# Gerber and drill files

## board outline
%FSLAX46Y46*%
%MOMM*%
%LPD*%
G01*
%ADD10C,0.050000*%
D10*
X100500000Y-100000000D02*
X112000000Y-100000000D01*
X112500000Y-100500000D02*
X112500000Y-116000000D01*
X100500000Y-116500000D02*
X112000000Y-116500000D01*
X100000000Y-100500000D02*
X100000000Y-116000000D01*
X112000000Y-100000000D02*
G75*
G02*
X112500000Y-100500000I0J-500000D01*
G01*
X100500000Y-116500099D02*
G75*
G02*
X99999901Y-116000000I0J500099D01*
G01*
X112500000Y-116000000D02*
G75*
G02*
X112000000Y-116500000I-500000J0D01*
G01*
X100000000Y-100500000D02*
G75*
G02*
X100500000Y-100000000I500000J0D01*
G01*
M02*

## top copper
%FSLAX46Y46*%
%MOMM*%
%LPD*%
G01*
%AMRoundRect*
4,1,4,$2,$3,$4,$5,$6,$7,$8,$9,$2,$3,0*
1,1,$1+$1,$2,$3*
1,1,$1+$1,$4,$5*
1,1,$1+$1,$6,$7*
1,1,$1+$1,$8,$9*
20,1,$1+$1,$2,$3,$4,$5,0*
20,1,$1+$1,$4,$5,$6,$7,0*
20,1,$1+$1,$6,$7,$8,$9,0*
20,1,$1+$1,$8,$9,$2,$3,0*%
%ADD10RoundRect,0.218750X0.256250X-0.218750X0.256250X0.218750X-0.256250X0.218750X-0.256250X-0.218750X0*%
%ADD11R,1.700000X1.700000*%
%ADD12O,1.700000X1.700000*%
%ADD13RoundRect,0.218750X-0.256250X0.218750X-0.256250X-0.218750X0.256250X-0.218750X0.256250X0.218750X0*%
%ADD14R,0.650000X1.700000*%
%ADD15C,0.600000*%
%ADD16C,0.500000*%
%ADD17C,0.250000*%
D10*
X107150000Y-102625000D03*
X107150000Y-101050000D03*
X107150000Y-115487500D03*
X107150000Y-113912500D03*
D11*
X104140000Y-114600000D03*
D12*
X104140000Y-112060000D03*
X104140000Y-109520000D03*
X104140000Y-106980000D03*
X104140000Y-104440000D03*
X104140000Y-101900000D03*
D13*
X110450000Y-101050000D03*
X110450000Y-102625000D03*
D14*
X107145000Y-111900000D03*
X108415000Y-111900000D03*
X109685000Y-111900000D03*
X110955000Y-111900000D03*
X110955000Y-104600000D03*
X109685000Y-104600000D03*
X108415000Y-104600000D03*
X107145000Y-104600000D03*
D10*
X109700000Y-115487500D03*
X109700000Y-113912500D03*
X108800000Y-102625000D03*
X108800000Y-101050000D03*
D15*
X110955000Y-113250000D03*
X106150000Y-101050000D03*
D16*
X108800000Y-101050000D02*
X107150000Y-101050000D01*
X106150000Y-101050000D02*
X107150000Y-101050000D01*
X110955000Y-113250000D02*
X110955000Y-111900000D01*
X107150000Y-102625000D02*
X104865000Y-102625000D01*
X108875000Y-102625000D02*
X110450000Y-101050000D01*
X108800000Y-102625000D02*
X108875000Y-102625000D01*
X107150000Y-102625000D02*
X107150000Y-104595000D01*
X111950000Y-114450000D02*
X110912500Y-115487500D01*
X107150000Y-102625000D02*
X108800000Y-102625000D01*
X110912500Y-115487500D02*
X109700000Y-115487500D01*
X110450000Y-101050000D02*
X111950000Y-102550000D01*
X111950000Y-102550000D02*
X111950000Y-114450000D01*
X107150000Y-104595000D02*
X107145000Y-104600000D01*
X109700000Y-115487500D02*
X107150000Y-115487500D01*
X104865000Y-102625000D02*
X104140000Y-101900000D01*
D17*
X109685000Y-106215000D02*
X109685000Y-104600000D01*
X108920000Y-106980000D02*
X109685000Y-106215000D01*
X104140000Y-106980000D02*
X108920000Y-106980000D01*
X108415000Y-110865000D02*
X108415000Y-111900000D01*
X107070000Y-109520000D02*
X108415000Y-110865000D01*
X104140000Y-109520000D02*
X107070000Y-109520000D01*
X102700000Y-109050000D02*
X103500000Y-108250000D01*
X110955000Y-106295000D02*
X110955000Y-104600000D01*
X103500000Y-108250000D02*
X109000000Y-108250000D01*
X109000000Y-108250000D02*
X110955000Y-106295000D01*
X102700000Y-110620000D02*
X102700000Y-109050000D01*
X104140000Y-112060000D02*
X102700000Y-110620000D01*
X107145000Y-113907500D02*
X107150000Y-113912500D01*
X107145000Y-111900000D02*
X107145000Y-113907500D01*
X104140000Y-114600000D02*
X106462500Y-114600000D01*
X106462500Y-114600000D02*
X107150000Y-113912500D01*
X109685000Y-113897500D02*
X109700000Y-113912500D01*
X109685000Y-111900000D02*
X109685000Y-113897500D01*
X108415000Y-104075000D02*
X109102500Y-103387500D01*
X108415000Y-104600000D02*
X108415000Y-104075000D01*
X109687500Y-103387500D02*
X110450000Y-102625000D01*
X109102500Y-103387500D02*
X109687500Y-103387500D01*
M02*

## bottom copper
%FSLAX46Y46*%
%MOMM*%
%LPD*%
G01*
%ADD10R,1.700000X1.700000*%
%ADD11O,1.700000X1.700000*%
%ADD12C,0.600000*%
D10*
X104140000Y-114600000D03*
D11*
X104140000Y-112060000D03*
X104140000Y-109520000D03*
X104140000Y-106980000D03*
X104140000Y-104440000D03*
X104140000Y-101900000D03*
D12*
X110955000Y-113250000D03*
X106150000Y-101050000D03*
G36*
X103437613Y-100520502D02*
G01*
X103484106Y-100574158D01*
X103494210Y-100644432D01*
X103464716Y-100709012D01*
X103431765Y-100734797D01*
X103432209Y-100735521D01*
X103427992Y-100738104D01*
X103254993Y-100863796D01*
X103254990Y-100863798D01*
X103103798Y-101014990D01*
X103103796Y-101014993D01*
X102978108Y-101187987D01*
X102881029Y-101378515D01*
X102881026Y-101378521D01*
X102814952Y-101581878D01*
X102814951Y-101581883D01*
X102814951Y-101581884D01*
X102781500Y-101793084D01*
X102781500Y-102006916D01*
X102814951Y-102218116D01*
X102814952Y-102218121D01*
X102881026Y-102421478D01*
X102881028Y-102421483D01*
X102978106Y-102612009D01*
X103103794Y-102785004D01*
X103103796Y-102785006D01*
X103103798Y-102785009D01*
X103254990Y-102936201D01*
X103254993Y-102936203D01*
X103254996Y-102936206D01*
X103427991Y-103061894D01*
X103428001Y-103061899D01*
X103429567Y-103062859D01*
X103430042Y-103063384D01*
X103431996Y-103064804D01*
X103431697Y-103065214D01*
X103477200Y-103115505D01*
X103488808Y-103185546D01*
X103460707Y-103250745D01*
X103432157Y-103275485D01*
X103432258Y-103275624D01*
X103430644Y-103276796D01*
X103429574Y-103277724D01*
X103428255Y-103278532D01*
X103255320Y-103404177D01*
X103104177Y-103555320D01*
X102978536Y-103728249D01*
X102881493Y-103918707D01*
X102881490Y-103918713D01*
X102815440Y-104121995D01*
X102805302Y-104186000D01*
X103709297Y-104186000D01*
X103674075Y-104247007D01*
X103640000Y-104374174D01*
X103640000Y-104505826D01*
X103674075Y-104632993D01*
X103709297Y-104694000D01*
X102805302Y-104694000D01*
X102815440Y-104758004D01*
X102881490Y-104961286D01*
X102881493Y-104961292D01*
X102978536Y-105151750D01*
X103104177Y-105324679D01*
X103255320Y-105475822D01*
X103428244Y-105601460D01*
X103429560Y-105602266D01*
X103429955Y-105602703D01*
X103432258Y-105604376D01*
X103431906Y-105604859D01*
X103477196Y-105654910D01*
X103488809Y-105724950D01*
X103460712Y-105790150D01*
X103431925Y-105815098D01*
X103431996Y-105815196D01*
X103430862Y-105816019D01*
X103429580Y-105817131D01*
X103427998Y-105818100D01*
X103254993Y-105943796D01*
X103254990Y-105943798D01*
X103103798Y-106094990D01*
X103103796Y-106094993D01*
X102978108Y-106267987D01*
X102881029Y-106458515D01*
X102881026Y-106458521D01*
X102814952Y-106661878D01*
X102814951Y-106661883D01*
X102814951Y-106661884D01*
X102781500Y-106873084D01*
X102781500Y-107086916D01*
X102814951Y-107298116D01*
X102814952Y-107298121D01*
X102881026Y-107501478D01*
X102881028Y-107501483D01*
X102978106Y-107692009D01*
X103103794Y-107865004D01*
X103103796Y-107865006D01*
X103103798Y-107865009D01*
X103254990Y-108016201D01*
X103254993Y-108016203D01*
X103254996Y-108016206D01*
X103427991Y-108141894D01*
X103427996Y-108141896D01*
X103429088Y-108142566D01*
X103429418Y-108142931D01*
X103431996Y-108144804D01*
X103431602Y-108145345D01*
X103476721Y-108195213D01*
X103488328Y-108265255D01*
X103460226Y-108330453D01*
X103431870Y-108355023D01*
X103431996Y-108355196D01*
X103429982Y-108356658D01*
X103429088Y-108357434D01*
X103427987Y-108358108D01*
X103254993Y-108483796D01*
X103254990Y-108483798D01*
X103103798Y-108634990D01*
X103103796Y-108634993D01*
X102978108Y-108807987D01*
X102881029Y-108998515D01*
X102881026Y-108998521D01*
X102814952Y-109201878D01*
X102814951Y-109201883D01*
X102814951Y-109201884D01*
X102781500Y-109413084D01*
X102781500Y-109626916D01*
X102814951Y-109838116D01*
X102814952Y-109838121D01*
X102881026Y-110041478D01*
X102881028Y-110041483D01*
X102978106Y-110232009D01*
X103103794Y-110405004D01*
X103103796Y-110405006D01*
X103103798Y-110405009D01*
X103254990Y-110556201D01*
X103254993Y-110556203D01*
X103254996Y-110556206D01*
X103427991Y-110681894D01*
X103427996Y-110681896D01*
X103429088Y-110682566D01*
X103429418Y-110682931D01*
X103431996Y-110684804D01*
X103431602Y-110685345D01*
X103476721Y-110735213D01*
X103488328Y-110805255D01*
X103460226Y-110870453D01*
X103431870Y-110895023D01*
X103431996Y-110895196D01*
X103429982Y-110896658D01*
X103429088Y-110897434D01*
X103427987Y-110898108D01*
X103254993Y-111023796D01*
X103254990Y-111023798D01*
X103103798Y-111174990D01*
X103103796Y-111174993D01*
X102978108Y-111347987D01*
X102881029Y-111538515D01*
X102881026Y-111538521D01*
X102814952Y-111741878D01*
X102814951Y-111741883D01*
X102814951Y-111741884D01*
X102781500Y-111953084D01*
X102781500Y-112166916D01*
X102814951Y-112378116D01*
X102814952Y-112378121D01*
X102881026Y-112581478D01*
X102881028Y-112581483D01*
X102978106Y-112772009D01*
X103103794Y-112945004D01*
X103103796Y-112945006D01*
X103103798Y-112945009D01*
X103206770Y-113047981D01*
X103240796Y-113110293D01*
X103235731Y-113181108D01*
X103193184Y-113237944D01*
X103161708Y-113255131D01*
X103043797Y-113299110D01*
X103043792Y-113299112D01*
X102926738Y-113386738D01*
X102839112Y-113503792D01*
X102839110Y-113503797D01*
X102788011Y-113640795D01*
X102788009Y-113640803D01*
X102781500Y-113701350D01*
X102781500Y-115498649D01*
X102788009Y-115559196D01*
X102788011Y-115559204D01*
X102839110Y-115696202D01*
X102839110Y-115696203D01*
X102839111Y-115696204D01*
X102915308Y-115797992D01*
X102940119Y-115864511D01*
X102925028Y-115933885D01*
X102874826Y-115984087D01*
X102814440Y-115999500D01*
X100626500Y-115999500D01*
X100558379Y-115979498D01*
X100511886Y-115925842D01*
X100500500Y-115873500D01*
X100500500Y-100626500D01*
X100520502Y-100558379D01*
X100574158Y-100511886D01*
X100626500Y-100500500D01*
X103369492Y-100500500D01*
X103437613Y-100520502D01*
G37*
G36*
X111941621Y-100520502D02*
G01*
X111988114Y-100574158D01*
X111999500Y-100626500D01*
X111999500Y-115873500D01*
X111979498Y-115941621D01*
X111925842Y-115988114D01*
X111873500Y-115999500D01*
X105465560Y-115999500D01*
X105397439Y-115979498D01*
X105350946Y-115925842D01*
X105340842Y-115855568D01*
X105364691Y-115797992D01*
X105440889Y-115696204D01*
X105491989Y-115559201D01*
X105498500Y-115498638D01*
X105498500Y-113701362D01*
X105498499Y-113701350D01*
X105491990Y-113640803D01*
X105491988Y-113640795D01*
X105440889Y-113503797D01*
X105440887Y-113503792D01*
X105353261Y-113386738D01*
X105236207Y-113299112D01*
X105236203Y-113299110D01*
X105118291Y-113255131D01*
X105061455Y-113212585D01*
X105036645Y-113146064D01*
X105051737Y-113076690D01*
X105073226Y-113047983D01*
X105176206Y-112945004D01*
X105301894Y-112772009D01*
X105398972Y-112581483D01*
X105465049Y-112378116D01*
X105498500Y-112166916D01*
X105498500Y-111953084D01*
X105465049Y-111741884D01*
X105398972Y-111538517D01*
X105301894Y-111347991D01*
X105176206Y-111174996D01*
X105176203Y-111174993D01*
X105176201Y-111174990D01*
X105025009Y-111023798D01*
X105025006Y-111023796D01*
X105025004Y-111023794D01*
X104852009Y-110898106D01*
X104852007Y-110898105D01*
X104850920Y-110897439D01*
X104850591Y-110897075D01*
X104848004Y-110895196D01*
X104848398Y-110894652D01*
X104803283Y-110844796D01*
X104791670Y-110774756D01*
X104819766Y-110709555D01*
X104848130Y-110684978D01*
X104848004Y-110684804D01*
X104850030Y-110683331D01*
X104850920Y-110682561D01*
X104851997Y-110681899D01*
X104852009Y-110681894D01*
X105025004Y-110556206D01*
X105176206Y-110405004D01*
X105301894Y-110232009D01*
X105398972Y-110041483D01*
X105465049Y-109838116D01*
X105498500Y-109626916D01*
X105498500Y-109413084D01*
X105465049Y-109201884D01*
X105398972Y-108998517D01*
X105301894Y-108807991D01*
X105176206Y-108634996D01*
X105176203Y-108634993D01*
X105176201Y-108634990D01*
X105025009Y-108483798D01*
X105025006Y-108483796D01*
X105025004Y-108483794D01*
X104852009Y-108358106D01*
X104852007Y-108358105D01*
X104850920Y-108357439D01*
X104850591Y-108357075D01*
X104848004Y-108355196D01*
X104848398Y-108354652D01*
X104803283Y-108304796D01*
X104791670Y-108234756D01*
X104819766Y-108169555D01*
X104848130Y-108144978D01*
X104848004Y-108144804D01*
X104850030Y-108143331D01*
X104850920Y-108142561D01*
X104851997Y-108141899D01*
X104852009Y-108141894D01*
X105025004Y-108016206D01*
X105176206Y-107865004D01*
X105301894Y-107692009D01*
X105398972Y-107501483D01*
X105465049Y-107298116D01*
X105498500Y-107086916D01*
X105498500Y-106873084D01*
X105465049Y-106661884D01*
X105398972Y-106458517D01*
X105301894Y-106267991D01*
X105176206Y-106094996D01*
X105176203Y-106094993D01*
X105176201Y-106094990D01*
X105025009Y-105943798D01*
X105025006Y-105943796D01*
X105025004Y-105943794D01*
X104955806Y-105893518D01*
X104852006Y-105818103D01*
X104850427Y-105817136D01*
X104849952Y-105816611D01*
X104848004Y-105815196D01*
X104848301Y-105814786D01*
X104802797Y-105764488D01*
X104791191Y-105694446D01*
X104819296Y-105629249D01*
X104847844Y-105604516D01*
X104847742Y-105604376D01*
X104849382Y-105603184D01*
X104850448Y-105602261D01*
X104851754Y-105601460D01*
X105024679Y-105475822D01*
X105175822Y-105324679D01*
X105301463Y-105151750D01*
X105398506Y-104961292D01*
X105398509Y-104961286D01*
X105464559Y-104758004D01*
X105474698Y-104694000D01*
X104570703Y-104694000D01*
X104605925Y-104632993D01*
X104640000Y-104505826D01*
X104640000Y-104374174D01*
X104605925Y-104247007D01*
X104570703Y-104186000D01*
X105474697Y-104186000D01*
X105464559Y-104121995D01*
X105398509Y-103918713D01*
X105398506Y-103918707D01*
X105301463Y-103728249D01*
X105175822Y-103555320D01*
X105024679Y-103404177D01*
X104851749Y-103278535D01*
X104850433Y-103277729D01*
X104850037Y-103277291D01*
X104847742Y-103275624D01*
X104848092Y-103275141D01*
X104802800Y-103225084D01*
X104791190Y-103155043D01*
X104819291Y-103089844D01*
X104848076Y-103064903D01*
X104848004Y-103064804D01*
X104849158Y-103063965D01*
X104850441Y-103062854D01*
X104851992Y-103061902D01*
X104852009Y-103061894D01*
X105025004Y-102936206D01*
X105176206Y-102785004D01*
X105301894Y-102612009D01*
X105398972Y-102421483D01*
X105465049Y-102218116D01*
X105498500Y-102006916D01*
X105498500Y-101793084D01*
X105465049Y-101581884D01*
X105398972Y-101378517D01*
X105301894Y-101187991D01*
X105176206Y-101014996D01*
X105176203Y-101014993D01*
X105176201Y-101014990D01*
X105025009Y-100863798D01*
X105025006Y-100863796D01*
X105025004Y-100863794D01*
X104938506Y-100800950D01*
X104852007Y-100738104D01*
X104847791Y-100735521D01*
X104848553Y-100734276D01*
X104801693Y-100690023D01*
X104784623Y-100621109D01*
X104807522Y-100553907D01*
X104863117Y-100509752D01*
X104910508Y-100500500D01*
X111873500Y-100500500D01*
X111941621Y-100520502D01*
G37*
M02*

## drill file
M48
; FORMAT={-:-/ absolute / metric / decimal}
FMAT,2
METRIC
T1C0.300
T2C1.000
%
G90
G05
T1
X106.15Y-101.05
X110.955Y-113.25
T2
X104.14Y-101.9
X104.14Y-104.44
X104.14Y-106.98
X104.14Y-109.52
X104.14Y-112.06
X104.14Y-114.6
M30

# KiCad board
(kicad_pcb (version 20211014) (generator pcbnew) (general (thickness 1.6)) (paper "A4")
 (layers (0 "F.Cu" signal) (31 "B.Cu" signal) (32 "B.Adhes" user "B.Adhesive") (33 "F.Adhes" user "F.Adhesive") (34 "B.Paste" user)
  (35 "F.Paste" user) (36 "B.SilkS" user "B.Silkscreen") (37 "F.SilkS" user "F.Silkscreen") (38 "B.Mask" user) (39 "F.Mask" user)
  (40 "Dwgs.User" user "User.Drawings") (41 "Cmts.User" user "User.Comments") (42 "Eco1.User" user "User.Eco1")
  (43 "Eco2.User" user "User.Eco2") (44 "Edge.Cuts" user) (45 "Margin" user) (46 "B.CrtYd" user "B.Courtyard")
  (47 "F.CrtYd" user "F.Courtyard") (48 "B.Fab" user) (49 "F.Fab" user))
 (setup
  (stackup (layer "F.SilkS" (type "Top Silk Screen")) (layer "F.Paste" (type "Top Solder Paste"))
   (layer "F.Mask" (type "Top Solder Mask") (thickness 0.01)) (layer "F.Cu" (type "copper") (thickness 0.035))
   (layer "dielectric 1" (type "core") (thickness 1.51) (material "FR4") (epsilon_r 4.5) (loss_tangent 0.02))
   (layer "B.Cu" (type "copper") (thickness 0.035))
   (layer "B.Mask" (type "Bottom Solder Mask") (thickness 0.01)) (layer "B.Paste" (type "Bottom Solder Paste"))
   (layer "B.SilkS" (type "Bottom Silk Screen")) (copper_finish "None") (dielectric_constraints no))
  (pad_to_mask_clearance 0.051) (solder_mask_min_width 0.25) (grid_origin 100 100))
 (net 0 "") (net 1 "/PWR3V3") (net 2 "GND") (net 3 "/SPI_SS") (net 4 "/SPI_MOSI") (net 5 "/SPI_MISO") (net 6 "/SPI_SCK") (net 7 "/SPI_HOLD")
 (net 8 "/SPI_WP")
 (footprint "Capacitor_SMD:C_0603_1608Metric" (layer "F.Cu") (at 107.15 101.8375 90)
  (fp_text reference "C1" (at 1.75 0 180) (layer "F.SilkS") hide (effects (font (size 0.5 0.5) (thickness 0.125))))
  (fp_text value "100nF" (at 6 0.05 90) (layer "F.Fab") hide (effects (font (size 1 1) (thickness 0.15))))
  (pad "1" smd roundrect locked (at -0.7875 0 90) (size 0.875 0.95) (layers "F.Cu" "F.Paste" "F.Mask") (roundrect_rratio 0.25)
   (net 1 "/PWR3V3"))
  (pad "2" smd roundrect locked (at 0.7875 0 90) (size 0.875 0.95) (layers "F.Cu" "F.Paste" "F.Mask") (roundrect_rratio 0.25) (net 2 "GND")))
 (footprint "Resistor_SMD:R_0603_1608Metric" (layer "F.Cu") (at 107.15 114.7 90)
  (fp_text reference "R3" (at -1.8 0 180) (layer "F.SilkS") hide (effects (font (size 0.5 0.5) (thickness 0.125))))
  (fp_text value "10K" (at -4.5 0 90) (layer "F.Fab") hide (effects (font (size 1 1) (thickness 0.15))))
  (pad "1" smd roundrect locked (at -0.7875 0 90) (size 0.875 0.95) (layers "F.Cu" "F.Paste" "F.Mask") (roundrect_rratio 0.25)
   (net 1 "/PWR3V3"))
  (pad "2" smd roundrect locked (at 0.7875 0 90) (size 0.875 0.95) (layers "F.Cu" "F.Paste" "F.Mask") (roundrect_rratio 0.25)
   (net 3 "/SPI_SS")))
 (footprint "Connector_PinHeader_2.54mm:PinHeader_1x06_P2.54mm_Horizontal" (layer "F.Cu") (at 104.14 114.6 180)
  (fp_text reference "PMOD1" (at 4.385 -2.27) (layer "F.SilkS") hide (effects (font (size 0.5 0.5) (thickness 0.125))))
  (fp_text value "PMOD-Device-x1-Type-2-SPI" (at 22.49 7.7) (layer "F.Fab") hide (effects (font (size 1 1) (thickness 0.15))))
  (pad "1" thru_hole rect locked (at 0 0 180) (size 1.7 1.7) (drill 1) (layers *.Cu *.Mask) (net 3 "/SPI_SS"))
  (pad "2" thru_hole oval locked (at 0 2.54 180) (size 1.7 1.7) (drill 1) (layers *.Cu *.Mask) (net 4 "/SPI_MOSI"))
  (pad "3" thru_hole oval locked (at 0 5.08 180) (size 1.7 1.7) (drill 1) (layers *.Cu *.Mask) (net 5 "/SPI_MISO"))
  (pad "4" thru_hole oval locked (at 0 7.62 180) (size 1.7 1.7) (drill 1) (layers *.Cu *.Mask) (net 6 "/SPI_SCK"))
  (pad "5" thru_hole oval locked (at 0 10.16 180) (size 1.7 1.7) (drill 1) (layers *.Cu *.Mask) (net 2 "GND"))
  (pad "6" thru_hole oval locked (at 0 12.7 180) (size 1.7 1.7) (drill 1) (layers *.Cu *.Mask) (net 1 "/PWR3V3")))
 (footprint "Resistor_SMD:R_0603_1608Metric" (layer "F.Cu") (at 110.45 101.8375 -90)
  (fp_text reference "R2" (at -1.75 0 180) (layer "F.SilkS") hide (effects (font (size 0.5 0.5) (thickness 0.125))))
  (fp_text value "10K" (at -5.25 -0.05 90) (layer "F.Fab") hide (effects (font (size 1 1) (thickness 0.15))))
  (pad "1" smd roundrect locked (at -0.7875 0 270) (size 0.875 0.95) (layers "F.Cu" "F.Paste" "F.Mask") (roundrect_rratio 0.25)
   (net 1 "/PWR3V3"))
  (pad "2" smd roundrect locked (at 0.7875 0 270) (size 0.875 0.95) (layers "F.Cu" "F.Paste" "F.Mask") (roundrect_rratio 0.25)
   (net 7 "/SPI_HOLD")))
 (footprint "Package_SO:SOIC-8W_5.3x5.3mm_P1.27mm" (layer "F.Cu") (at 109.05 108.25 90)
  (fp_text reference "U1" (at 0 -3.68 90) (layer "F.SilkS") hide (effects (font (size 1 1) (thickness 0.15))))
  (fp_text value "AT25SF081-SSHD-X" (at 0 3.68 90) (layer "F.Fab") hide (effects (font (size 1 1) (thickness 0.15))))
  (pad "1" smd rect (at -3.65 -1.905 90) (size 1.7 0.65) (layers "F.Cu" "F.Paste" "F.Mask") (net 3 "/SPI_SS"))
  (pad "2" smd rect (at -3.65 -0.635 90) (size 1.7 0.65) (layers "F.Cu" "F.Paste" "F.Mask") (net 5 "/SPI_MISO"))
  (pad "3" smd rect (at -3.65 0.635 90) (size 1.7 0.65) (layers "F.Cu" "F.Paste" "F.Mask") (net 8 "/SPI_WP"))
  (pad "4" smd rect (at -3.65 1.905 90) (size 1.7 0.65) (layers "F.Cu" "F.Paste" "F.Mask") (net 2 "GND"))
  (pad "5" smd rect (at 3.65 1.905 90) (size 1.7 0.65) (layers "F.Cu" "F.Paste" "F.Mask") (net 4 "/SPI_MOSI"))
  (pad "6" smd rect (at 3.65 0.635 90) (size 1.7 0.65) (layers "F.Cu" "F.Paste" "F.Mask") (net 6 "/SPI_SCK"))
  (pad "7" smd rect (at 3.65 -0.635 90) (size 1.7 0.65) (layers "F.Cu" "F.Paste" "F.Mask") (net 7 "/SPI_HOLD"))
  (pad "8" smd rect (at 3.65 -1.905 90) (size 1.7 0.65) (layers "F.Cu" "F.Paste" "F.Mask") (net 1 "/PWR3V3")))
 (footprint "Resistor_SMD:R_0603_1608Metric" (layer "F.Cu") (at 109.7 114.7 90)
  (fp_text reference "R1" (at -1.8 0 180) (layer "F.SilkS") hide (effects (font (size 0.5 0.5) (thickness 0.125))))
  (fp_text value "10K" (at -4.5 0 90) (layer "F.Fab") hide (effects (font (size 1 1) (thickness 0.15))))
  (pad "1" smd roundrect locked (at -0.7875 0 90) (size 0.875 0.95) (layers "F.Cu" "F.Paste" "F.Mask") (roundrect_rratio 0.25)
   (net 1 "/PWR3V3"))
  (pad "2" smd roundrect locked (at 0.7875 0 90) (size 0.875 0.95) (layers "F.Cu" "F.Paste" "F.Mask") (roundrect_rratio 0.25)
   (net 8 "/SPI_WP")))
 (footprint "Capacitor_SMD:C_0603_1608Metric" (layer "F.Cu") (at 108.8 101.8375 90)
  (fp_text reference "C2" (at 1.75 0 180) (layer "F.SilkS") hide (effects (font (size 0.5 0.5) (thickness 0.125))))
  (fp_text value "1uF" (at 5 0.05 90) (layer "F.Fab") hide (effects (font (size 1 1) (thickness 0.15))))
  (pad "1" smd roundrect locked (at -0.7875 0 90) (size 0.875 0.95) (layers "F.Cu" "F.Paste" "F.Mask") (roundrect_rratio 0.25)
   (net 1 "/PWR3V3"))
  (pad "2" smd roundrect locked (at 0.7875 0 90) (size 0.875 0.95) (layers "F.Cu" "F.Paste" "F.Mask") (roundrect_rratio 0.25) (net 2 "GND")))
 (gr_line (start 100.5 100) (end 112 100) (layer "Edge.Cuts") (width 0.05))
 (gr_line (start 112.5 100.5) (end 112.5 116) (layer "Edge.Cuts") (width 0.05))
 (gr_line (start 100.5 116.5) (end 112 116.5) (layer "Edge.Cuts") (width 0.05))
 (gr_line (start 100 100.5) (end 100 116) (layer "Edge.Cuts") (width 0.05))
 (gr_arc (start 112 100) (mid 112.353553 100.146447) (end 112.5 100.5) (layer "Edge.Cuts") (width 0.05))
 (gr_arc (start 100.5 116.500099) (mid 100.146377 116.353623) (end 99.999901 116) (layer "Edge.Cuts") (width 0.05))
 (gr_arc (start 112.5 116) (mid 112.353553 116.353553) (end 112 116.5) (layer "Edge.Cuts") (width 0.05))
 (gr_arc (start 100 100.5) (mid 100.146447 100.146447) (end 100.5 100) (layer "Edge.Cuts") (width 0.05))
 (segment (start 108.8 101.05) (end 107.15 101.05) (width 0.5) (layer "F.Cu") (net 2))
 (segment (start 106.15 101.05) (end 107.15 101.05) (width 0.5) (layer "F.Cu") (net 2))
 (segment (start 110.955 113.25) (end 110.955 111.9) (width 0.5) (layer "F.Cu") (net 2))
 (via (at 110.955 113.25) (size 0.6) (drill 0.3) (layers "F.Cu" "B.Cu") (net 2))
 (via (at 106.15 101.05) (size 0.6) (drill 0.3) (layers "F.Cu" "B.Cu") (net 2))
 (segment (start 107.15 102.625) (end 104.865 102.625) (width 0.5) (layer "F.Cu") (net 1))
 (segment (start 108.875 102.625) (end 110.45 101.05) (width 0.5) (layer "F.Cu") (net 1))
 (segment (start 108.8 102.625) (end 108.875 102.625) (width 0.5) (layer "F.Cu") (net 1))
 (segment (start 107.15 102.625) (end 107.15 104.595) (width 0.5) (layer "F.Cu") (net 1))
 (segment (start 111.95 114.45) (end 110.9125 115.4875) (width 0.5) (layer "F.Cu") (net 1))
 (segment (start 107.15 102.625) (end 108.8 102.625) (width 0.5) (layer "F.Cu") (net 1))
 (segment (start 110.9125 115.4875) (end 109.7 115.4875) (width 0.5) (layer "F.Cu") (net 1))
 (segment (start 110.45 101.05) (end 111.95 102.55) (width 0.5) (layer "F.Cu") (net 1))
 (segment (start 111.95 102.55) (end 111.95 114.45) (width 0.5) (layer "F.Cu") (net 1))
 (segment (start 107.15 104.595) (end 107.145 104.6) (width 0.5) (layer "F.Cu") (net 1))
 (segment (start 109.7 115.4875) (end 107.15 115.4875) (width 0.5) (layer "F.Cu") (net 1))
 (segment (start 104.865 102.625) (end 104.14 101.9) (width 0.5) (layer "F.Cu") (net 1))
 (segment (start 109.685 106.215) (end 109.685 104.6) (width 0.25) (layer "F.Cu") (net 6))
 (segment (start 108.92 106.98) (end 109.685 106.215) (width 0.25) (layer "F.Cu") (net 6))
 (segment (start 104.14 106.98) (end 108.92 106.98) (width 0.25) (layer "F.Cu") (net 6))
 (segment (start 108.415 110.865) (end 108.415 111.9) (width 0.25) (layer "F.Cu") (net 5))
 (segment (start 107.07 109.52) (end 108.415 110.865) (width 0.25) (layer "F.Cu") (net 5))
 (segment (start 104.14 109.52) (end 107.07 109.52) (width 0.25) (layer "F.Cu") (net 5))
 (segment (start 102.7 109.05) (end 103.5 108.25) (width 0.25) (layer "F.Cu") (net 4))
 (segment (start 110.955 106.295) (end 110.955 104.6) (width 0.25) (layer "F.Cu") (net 4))
 (segment (start 103.5 108.25) (end 109 108.25) (width 0.25) (layer "F.Cu") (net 4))
 (segment (start 109 108.25) (end 110.955 106.295) (width 0.25) (layer "F.Cu") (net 4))
 (segment (start 102.7 110.62) (end 102.7 109.05) (width 0.25) (layer "F.Cu") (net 4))
 (segment (start 104.14 112.06) (end 102.7 110.62) (width 0.25) (layer "F.Cu") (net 4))
 (segment (start 107.145 113.9075) (end 107.15 113.9125) (width 0.25) (layer "F.Cu") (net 3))
 (segment (start 107.145 111.9) (end 107.145 113.9075) (width 0.25) (layer "F.Cu") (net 3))
 (segment (start 104.14 114.6) (end 106.4625 114.6) (width 0.25) (layer "F.Cu") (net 3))
 (segment (start 106.4625 114.6) (end 107.15 113.9125) (width 0.25) (layer "F.Cu") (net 3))
 (segment (start 109.685 113.8975) (end 109.7 113.9125) (width 0.25) (layer "F.Cu") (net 8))
 (segment (start 109.685 111.9) (end 109.685 113.8975) (width 0.25) (layer "F.Cu") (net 8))
 (segment (start 108.415 104.075) (end 109.1025 103.3875) (width 0.25) (layer "F.Cu") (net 7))
 (segment (start 108.415 104.6) (end 108.415 104.075) (width 0.25) (layer "F.Cu") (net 7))
 (segment (start 109.6875 103.3875) (end 110.45 102.625) (width 0.25) (layer "F.Cu") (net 7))
 (segment (start 109.1025 103.3875) (end 109.6875 103.3875) (width 0.25) (layer "F.Cu") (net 7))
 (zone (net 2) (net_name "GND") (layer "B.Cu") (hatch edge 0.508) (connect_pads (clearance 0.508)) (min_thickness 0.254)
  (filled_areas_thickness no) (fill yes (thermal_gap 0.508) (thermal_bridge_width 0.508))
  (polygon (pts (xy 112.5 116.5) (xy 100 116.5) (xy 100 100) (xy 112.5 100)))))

